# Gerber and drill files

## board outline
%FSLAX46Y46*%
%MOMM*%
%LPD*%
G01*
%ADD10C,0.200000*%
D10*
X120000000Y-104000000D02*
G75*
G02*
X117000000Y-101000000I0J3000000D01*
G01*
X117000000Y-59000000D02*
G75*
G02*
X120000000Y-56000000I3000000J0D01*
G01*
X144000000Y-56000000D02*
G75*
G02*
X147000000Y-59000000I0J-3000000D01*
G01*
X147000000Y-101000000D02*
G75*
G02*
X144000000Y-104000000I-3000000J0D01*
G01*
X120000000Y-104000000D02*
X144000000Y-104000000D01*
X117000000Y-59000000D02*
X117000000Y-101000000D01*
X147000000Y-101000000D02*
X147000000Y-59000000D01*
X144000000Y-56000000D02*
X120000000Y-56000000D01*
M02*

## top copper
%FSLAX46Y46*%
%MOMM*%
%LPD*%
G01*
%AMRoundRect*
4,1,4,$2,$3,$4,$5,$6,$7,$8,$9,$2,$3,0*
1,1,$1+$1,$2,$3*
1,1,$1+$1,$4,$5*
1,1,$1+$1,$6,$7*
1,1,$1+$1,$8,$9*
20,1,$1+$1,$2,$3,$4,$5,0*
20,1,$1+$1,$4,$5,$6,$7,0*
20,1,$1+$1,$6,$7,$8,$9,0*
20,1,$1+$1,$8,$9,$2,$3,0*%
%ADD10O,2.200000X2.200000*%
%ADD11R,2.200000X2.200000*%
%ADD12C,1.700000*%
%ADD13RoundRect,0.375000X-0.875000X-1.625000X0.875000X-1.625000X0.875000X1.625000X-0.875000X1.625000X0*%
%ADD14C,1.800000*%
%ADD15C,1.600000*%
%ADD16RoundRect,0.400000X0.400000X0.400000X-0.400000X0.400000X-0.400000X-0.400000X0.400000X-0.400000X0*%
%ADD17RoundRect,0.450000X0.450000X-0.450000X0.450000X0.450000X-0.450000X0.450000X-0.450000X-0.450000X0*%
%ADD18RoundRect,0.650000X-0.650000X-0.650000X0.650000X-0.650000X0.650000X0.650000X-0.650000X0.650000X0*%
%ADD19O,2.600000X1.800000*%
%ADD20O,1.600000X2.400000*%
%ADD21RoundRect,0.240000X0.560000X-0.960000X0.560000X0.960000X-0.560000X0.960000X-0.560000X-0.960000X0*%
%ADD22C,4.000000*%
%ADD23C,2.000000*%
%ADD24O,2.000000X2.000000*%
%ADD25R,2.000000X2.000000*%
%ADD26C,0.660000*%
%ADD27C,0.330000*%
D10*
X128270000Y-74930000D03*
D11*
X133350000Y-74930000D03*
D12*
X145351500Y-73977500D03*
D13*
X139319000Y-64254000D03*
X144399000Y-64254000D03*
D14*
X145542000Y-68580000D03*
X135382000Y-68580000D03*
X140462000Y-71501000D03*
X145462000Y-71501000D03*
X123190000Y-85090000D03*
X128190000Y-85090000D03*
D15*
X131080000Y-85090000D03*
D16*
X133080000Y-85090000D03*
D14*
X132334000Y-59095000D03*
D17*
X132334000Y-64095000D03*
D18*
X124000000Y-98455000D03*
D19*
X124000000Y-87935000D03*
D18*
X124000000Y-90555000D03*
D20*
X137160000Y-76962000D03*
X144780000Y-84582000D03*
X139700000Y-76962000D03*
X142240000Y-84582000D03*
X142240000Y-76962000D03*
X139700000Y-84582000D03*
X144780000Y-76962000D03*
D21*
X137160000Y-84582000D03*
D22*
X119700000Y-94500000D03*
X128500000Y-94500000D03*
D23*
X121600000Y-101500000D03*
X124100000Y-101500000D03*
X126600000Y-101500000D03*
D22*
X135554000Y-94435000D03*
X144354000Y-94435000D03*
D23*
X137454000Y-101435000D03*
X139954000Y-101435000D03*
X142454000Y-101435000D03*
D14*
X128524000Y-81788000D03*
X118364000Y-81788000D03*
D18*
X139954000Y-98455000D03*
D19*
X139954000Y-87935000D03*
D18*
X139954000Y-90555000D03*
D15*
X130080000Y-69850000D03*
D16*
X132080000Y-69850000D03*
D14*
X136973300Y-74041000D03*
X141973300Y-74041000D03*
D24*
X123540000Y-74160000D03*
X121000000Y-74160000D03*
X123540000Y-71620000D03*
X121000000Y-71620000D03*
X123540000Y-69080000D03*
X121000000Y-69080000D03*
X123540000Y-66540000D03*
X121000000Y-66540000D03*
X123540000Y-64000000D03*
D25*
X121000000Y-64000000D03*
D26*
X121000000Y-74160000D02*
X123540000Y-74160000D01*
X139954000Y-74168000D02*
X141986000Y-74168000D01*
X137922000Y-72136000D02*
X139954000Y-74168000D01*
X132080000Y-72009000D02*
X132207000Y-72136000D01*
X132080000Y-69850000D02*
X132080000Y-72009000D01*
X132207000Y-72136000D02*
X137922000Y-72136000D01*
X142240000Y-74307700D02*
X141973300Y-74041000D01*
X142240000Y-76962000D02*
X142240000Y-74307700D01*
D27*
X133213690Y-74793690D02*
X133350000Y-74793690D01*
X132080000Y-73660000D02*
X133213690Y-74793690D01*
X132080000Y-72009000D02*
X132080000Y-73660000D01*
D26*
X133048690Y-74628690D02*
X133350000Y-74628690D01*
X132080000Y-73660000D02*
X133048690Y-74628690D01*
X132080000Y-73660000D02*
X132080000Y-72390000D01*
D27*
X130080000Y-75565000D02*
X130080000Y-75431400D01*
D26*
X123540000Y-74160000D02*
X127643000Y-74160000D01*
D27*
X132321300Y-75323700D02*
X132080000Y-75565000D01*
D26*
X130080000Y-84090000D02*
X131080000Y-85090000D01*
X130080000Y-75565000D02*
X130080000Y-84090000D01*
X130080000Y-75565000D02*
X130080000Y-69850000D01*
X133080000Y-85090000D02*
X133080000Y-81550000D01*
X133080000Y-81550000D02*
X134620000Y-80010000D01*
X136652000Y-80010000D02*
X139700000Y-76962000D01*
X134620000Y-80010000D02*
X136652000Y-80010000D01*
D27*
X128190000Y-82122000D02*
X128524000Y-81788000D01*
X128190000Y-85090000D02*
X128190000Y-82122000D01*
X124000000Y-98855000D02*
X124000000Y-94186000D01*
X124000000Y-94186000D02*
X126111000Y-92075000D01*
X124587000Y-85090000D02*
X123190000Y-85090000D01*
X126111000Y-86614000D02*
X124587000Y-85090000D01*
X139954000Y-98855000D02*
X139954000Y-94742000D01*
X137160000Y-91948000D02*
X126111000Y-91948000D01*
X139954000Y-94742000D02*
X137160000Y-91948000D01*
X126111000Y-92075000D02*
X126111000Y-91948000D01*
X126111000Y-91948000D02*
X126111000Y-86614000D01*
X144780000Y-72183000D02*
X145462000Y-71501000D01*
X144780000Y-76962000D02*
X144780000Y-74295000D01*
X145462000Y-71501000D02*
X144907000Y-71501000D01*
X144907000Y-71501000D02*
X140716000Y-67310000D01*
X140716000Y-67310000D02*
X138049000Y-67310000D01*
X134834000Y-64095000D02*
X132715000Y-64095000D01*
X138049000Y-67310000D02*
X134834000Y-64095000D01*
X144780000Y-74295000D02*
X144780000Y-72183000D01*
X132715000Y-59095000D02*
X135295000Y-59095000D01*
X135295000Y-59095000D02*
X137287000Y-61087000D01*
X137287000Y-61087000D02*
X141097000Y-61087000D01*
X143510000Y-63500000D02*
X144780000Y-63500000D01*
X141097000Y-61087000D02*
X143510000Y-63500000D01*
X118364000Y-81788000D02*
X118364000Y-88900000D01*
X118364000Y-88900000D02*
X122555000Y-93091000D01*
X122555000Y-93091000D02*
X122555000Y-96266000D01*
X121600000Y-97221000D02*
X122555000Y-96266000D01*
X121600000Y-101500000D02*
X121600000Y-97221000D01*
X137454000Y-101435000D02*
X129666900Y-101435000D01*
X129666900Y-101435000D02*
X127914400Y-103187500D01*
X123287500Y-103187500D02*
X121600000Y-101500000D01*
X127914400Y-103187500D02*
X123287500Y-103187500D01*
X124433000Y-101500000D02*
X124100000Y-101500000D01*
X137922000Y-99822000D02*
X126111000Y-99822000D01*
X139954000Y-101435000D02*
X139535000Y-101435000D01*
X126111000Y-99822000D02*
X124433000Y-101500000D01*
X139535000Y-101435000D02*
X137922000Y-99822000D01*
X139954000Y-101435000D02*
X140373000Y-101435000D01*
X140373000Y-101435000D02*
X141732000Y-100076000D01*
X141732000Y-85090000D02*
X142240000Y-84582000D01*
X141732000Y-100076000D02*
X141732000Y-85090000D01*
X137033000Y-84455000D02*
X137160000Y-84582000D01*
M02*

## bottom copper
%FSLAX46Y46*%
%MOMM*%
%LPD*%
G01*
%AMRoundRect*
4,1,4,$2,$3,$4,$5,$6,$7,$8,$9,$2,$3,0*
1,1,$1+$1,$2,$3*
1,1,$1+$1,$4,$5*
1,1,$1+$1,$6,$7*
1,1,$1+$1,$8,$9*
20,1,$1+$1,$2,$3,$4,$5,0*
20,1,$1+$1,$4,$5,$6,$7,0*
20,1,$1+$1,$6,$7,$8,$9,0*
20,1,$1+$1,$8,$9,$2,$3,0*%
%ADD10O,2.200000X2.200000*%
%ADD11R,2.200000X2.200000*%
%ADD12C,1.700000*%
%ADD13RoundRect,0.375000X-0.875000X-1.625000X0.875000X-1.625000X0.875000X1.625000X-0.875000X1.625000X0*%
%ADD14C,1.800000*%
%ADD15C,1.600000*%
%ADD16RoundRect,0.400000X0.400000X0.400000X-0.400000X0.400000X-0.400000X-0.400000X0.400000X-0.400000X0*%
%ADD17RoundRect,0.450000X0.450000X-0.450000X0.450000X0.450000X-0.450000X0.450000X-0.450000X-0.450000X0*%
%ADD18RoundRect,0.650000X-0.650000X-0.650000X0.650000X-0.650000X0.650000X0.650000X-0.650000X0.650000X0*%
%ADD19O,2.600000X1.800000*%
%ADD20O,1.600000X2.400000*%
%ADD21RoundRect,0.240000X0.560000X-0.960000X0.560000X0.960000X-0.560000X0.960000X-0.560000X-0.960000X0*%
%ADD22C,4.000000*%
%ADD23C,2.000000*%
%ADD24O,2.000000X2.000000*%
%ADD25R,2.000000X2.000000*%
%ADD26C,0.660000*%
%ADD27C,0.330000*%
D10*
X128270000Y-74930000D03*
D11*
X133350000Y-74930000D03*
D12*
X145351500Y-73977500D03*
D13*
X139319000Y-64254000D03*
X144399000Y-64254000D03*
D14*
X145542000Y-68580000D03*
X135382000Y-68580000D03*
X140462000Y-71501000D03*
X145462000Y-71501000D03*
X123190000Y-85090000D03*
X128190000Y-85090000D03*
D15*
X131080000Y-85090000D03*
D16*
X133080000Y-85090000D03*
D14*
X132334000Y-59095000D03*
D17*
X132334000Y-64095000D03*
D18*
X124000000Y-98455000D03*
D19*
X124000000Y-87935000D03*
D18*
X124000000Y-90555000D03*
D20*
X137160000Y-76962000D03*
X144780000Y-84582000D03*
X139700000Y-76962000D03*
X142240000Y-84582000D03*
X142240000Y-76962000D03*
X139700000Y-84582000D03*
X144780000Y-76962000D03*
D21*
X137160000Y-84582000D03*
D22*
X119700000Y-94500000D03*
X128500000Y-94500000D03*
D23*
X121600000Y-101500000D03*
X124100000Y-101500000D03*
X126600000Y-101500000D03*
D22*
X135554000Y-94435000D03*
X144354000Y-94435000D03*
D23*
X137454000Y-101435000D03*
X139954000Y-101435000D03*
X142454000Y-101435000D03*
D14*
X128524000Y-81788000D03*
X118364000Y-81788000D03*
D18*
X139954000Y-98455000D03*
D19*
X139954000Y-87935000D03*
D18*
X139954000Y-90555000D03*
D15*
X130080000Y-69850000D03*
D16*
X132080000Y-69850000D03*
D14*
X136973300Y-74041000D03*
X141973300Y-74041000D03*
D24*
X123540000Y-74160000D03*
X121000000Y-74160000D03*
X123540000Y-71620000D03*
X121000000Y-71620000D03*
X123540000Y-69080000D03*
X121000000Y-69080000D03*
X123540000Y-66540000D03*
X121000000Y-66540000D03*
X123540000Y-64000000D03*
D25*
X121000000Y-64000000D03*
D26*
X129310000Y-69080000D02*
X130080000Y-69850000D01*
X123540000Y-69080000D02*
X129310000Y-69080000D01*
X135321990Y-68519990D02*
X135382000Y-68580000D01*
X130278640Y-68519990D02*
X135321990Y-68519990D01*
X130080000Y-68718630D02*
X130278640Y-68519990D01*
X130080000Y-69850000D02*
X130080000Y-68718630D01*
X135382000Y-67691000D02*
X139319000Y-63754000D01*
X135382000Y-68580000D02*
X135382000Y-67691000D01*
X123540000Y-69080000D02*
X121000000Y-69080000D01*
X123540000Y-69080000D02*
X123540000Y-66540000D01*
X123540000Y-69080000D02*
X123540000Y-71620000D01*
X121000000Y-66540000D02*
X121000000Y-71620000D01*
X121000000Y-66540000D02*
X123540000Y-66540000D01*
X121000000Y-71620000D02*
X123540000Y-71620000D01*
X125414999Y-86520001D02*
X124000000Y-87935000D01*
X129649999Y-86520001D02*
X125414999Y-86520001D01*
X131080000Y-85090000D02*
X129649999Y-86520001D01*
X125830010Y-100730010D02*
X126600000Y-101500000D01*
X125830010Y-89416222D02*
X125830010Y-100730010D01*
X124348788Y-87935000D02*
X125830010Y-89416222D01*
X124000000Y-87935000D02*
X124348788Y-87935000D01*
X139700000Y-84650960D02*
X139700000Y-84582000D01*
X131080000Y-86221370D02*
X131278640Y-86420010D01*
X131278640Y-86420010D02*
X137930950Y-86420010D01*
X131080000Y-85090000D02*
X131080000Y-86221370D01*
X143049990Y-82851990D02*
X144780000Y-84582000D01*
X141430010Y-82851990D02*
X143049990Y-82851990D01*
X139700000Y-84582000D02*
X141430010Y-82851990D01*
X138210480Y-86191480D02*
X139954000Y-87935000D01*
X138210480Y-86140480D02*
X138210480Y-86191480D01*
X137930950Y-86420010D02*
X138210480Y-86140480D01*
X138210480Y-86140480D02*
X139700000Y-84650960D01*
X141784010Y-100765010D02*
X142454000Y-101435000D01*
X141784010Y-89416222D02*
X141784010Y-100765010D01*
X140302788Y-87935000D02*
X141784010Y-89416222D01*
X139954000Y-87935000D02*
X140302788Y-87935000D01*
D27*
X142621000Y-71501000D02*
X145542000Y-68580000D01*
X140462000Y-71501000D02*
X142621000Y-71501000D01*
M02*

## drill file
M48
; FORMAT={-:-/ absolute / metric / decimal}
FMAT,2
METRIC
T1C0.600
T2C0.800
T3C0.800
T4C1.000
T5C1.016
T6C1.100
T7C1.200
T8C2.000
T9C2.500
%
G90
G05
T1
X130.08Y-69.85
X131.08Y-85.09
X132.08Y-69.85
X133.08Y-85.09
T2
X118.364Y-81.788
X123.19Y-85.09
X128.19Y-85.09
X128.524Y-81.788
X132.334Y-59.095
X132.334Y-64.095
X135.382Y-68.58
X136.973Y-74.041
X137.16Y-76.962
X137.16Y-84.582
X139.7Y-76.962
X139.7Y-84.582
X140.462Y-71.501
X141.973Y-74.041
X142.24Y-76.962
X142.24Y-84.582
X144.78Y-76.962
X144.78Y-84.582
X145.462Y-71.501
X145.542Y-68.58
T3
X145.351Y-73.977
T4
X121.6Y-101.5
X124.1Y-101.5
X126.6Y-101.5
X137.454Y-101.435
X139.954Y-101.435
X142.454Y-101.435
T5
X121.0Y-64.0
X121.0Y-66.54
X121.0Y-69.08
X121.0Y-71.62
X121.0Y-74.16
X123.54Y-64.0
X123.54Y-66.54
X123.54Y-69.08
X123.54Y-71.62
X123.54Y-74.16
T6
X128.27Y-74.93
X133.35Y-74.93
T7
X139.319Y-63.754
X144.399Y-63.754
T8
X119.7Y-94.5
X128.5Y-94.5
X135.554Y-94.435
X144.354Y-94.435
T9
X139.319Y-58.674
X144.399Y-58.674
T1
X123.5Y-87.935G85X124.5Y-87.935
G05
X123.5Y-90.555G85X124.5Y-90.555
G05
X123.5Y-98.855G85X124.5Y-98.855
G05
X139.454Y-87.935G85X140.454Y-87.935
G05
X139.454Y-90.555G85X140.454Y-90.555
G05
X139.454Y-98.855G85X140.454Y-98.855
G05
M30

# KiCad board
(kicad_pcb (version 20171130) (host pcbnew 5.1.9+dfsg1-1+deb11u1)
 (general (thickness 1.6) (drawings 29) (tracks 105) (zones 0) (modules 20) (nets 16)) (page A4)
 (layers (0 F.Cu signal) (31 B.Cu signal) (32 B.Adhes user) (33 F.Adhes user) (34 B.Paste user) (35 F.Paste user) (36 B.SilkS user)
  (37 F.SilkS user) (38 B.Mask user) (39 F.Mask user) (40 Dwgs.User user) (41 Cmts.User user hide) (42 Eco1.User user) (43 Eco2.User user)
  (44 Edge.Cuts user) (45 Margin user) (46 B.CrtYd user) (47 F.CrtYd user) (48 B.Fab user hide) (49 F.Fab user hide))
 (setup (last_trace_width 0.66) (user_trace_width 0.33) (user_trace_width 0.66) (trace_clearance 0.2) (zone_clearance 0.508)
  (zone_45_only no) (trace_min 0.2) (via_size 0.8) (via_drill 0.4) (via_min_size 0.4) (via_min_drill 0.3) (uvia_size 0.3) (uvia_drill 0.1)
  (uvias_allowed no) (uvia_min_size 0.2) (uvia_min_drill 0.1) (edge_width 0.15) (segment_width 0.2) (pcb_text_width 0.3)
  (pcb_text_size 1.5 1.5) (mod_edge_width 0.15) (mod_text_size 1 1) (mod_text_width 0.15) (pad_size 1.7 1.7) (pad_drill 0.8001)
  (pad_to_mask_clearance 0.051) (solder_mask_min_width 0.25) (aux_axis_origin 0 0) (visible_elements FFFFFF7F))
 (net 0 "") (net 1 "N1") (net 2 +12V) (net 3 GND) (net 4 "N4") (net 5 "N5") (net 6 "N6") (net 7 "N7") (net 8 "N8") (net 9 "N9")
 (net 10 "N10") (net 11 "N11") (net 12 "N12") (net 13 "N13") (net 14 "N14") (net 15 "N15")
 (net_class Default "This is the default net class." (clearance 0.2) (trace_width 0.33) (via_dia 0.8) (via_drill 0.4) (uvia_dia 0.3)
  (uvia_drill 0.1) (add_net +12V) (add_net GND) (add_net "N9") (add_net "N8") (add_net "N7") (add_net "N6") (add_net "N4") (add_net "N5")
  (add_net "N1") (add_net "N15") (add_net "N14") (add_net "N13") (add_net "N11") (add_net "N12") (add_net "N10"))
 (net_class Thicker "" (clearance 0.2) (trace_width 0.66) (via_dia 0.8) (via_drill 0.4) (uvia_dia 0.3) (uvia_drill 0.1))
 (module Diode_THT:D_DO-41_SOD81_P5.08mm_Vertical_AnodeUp (layer F.Cu) (at 133.35 74.93 180)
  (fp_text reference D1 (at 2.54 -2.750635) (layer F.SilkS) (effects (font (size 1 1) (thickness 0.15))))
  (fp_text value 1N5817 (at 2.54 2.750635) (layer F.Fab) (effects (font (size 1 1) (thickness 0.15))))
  (pad 2 thru_hole oval (at 5.08 0 180) (size 2.2 2.2) (drill 1.1) (layers *.Cu *.Mask) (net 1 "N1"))
  (pad 1 thru_hole rect (at 0 0 180) (size 2.2 2.2) (drill 1.1) (layers *.Cu *.Mask) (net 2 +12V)))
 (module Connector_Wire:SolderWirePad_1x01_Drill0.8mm (layer F.Cu) (at 145.3515 73.9775)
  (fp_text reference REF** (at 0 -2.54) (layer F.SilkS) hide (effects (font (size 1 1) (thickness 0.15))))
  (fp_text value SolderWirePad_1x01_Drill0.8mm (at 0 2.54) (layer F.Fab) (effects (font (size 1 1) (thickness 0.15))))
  (pad 1 thru_hole circle (at 0 0) (size 1.7 1.7) (drill 0.8001) (layers *.Cu *.Mask)))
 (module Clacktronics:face (layer B.Cu) (at 140.843 80.772 180)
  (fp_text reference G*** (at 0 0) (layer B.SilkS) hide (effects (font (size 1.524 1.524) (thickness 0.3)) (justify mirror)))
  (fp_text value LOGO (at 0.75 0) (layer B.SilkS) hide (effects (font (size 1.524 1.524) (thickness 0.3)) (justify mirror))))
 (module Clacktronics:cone (layer B.Cu) (at 122.047 60.579 180)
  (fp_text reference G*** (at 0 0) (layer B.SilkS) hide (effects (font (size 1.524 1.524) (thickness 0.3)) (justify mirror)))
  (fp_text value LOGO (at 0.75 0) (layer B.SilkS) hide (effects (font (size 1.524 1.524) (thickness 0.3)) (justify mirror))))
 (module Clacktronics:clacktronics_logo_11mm (layer F.Cu) (at 131.572 87.63)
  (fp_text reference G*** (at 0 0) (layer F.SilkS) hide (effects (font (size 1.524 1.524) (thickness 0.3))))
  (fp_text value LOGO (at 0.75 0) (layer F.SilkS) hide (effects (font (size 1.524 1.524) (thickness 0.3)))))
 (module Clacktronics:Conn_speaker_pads (layer F.Cu) (at 141.859 63.754)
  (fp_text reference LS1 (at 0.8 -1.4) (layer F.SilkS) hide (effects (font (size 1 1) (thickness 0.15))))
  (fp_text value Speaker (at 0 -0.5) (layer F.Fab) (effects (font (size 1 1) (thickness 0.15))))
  (pad 2 thru_hole roundrect (at -2.54 0) (size 2.5 4) (drill 1.2 (offset 0 0.5)) (layers *.Cu *.Mask) (roundrect_rratio 0.15) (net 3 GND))
  (pad "" np_thru_hole circle (at -2.54 -5.08) (size 2.5 2.5) (drill 2.5) (layers *.Cu *.Mask))
  (pad 1 thru_hole roundrect (at 2.54 0) (size 2.5 4) (drill 1.2 (offset 0 0.5)) (layers *.Cu *.Mask) (roundrect_rratio 0.15) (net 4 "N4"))
  (pad "" np_thru_hole circle (at 2.54 -5.08) (size 2.5 2.5) (drill 2.5) (layers *.Cu *.Mask)))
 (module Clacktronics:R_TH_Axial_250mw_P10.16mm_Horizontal (layer F.Cu) (at 135.382 68.58)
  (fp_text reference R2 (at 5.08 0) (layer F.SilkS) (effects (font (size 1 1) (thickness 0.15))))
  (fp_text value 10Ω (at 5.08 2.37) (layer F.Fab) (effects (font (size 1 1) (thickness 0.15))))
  (pad 2 thru_hole circle (at 10.16 0) (size 1.8 1.8) (drill 0.8) (layers *.Cu *.Mask) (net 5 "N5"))
  (pad 1 thru_hole circle (at 0 0) (size 1.8 1.8) (drill 0.8) (layers *.Cu *.Mask) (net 3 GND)))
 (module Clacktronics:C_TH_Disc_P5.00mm (layer F.Cu) (at 145.462 71.501 180)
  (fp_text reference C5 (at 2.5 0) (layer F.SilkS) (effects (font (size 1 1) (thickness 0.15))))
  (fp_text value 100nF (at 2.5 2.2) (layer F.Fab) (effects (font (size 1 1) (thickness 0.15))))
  (pad 2 thru_hole circle (at 5 0 180) (size 1.8 1.8) (drill 0.8) (layers *.Cu *.Mask) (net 5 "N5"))
  (pad 1 thru_hole circle (at 0 0 180) (size 1.8 1.8) (drill 0.8) (layers *.Cu *.Mask) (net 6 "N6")))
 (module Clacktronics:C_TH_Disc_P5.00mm (layer F.Cu) (at 128.19 85.09 180)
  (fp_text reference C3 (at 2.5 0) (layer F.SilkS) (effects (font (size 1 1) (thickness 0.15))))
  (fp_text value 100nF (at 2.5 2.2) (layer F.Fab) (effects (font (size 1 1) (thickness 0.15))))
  (pad 2 thru_hole circle (at 5 0 180) (size 1.8 1.8) (drill 0.8) (layers *.Cu *.Mask) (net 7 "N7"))
  (pad 1 thru_hole circle (at 0 0 180) (size 1.8 1.8) (drill 0.8) (layers *.Cu *.Mask) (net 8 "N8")))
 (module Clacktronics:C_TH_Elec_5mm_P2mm (layer F.Cu) (at 132.08 85.09 180)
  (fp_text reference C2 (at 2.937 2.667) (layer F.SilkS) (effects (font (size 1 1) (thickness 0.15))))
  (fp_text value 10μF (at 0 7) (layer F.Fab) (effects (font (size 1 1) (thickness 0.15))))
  (pad 2 thru_hole circle (at 1 0 180) (size 1.6 1.6) (drill 0.6) (layers *.Cu *.Mask) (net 3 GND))
  (pad 1 thru_hole roundrect (at -1 0 180) (size 1.6 1.6) (drill 0.6) (layers *.Cu *.Mask) (roundrect_rratio 0.25) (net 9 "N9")))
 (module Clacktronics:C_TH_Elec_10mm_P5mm (layer F.Cu) (at 132.334 61.595 90)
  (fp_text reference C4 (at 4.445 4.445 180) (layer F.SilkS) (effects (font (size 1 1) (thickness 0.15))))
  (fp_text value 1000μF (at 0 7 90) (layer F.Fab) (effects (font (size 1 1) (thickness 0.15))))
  (pad 2 thru_hole circle (at 2.5 0 90) (size 1.8 1.8) (drill 0.8) (layers *.Cu *.Mask) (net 4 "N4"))
  (pad 1 thru_hole roundrect (at -2.5 0 90) (size 1.8 1.8) (drill 0.8) (layers *.Cu *.Mask) (roundrect_rratio 0.25) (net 6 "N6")))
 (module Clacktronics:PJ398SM (layer B.Cu) (at 124 93.935 180)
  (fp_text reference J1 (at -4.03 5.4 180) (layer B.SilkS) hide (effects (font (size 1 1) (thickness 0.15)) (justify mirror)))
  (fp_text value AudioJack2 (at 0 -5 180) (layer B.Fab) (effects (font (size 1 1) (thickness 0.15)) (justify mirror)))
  (pad T thru_hole roundrect (at 0 -4.92) (size 2.6 2.6) (drill oval 1.6 0.6 (offset 0 -0.4)) (layers *.Cu *.Mask) (roundrect_rratio 0.25)
   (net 7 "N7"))
  (pad S thru_hole oval (at 0 6) (size 2.6 1.8) (drill oval 1.6 0.6) (layers *.Cu *.Mask) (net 3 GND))
  (pad TN thru_hole roundrect (at 0 3.38) (size 2.6 2.6) (drill oval 1.6 0.6) (layers *.Cu *.Mask) (roundrect_rratio 0.25)))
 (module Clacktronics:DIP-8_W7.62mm (layer F.Cu) (at 137.16 84.582 90)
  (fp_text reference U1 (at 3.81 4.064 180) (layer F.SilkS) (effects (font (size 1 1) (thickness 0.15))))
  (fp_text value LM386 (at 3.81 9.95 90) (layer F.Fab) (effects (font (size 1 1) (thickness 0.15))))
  (pad 8 thru_hole oval (at 7.62 0 90) (size 2.4 1.6) (drill 0.8) (layers *.Cu *.Mask) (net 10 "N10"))
  (pad 4 thru_hole oval (at 0 7.62 90) (size 2.4 1.6) (drill 0.8) (layers *.Cu *.Mask) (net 3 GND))
  (pad 7 thru_hole oval (at 7.62 2.54 90) (size 2.4 1.6) (drill 0.8) (layers *.Cu *.Mask) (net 9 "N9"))
  (pad 3 thru_hole oval (at 0 5.08 90) (size 2.4 1.6) (drill 0.8) (layers *.Cu *.Mask) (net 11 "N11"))
  (pad 6 thru_hole oval (at 7.62 5.08 90) (size 2.4 1.6) (drill 0.8) (layers *.Cu *.Mask) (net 2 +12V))
  (pad 2 thru_hole oval (at 0 2.54 90) (size 2.4 1.6) (drill 0.8) (layers *.Cu *.Mask) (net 3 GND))
  (pad 5 thru_hole oval (at 7.62 7.62 90) (size 2.4 1.6) (drill 0.8) (layers *.Cu *.Mask) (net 6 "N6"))
  (pad 1 thru_hole roundrect (at 0 0 90) (size 2.4 1.6) (drill 0.8) (layers *.Cu *.Mask) (roundrect_rratio 0.15) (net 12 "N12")))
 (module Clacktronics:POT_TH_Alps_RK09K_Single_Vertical (layer B.Cu) (at 124.1 94 180)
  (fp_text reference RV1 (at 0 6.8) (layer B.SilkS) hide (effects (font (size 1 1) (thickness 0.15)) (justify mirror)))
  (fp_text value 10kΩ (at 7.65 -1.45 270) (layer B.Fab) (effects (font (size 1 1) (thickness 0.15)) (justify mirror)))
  (pad "" thru_hole circle (at 4.4 -0.5 90) (size 4 4) (drill 2) (layers *.Cu *.Mask))
  (pad "" thru_hole circle (at -4.4 -0.5 90) (size 4 4) (drill 2) (layers *.Cu *.Mask))
  (pad 1 thru_hole circle (at 2.5 -7.5 90) (size 2 2) (drill 1) (layers *.Cu *.Mask) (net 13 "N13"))
  (pad 2 thru_hole circle (at 0 -7.5 180) (size 2 2) (drill 1) (layers *.Cu *.Mask) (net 11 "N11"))
  (pad 3 thru_hole circle (at -2.5 -7.5 90) (size 2 2) (drill 1) (layers *.Cu *.Mask) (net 3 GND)))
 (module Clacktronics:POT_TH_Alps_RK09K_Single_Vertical (layer B.Cu) (at 139.954 93.935 180)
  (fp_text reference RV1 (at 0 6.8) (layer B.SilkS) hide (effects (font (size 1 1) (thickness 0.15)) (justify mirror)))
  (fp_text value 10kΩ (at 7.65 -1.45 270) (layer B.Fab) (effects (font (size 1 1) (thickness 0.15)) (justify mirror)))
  (pad "" thru_hole circle (at 4.4 -0.5 90) (size 4 4) (drill 2) (layers *.Cu *.Mask))
  (pad "" thru_hole circle (at -4.4 -0.5 90) (size 4 4) (drill 2) (layers *.Cu *.Mask))
  (pad 1 thru_hole circle (at 2.5 -7.5 90) (size 2 2) (drill 1) (layers *.Cu *.Mask) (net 13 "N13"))
  (pad 2 thru_hole circle (at 0 -7.5 180) (size 2 2) (drill 1) (layers *.Cu *.Mask) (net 11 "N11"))
  (pad 3 thru_hole circle (at -2.5 -7.5 90) (size 2 2) (drill 1) (layers *.Cu *.Mask) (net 3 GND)))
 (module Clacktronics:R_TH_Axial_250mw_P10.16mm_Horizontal (layer F.Cu) (at 118.364 81.788)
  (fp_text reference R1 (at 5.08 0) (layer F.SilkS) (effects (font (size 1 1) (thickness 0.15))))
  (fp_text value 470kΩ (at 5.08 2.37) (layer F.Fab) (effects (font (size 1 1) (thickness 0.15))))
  (pad 2 thru_hole circle (at 10.16 0) (size 1.8 1.8) (drill 0.8) (layers *.Cu *.Mask) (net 8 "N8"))
  (pad 1 thru_hole circle (at 0 0) (size 1.8 1.8) (drill 0.8) (layers *.Cu *.Mask) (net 13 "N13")))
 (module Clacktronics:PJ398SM (layer B.Cu) (at 139.954 93.935 180)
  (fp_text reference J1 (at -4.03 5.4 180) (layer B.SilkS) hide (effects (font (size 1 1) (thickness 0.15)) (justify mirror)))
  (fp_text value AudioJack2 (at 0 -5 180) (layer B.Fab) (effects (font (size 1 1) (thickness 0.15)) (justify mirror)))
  (pad T thru_hole roundrect (at 0 -4.92) (size 2.6 2.6) (drill oval 1.6 0.6 (offset 0 -0.4)) (layers *.Cu *.Mask) (roundrect_rratio 0.25)
   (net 7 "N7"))
  (pad S thru_hole oval (at 0 6) (size 2.6 1.8) (drill oval 1.6 0.6) (layers *.Cu *.Mask) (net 3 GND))
  (pad TN thru_hole roundrect (at 0 3.38) (size 2.6 2.6) (drill oval 1.6 0.6) (layers *.Cu *.Mask) (roundrect_rratio 0.25)))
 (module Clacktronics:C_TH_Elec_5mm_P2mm (layer F.Cu) (at 131.08 69.85 180)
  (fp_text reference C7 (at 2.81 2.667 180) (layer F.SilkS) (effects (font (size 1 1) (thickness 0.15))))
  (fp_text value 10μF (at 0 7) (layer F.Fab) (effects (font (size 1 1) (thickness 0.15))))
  (pad 2 thru_hole circle (at 1 0 180) (size 1.6 1.6) (drill 0.6) (layers *.Cu *.Mask) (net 3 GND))
  (pad 1 thru_hole roundrect (at -1 0 180) (size 1.6 1.6) (drill 0.6) (layers *.Cu *.Mask) (roundrect_rratio 0.25) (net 2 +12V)))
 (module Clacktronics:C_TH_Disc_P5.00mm (layer F.Cu) (at 141.9733 74.041 180)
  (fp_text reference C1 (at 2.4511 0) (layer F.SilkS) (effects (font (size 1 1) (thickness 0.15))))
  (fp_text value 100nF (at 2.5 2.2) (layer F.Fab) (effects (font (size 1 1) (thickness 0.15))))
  (pad 2 thru_hole circle (at 5 0 180) (size 1.8 1.8) (drill 0.8) (layers *.Cu *.Mask) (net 3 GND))
  (pad 1 thru_hole circle (at 0 0 180) (size 1.8 1.8) (drill 0.8) (layers *.Cu *.Mask) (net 2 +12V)))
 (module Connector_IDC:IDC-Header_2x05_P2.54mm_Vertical (layer F.Cu) (at 121 64)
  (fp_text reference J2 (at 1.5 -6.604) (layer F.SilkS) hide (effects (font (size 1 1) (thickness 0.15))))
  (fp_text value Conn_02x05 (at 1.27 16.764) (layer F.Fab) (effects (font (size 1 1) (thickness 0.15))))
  (pad 10 thru_hole oval (at 2.54 10.16) (size 2 2) (drill 1.016) (layers *.Cu *.Mask) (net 1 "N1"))
  (pad 9 thru_hole oval (at 0 10.16) (size 2 2) (drill 1.016) (layers *.Cu *.Mask) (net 1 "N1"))
  (pad 8 thru_hole oval (at 2.54 7.62) (size 2 2) (drill 1.016) (layers *.Cu *.Mask) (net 3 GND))
  (pad 7 thru_hole oval (at 0 7.62) (size 2 2) (drill 1.016) (layers *.Cu *.Mask) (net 3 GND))
  (pad 6 thru_hole oval (at 2.54 5.08) (size 2 2) (drill 1.016) (layers *.Cu *.Mask) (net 3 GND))
  (pad 5 thru_hole oval (at 0 5.08) (size 2 2) (drill 1.016) (layers *.Cu *.Mask) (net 3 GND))
  (pad 4 thru_hole oval (at 2.54 2.54) (size 2 2) (drill 1.016) (layers *.Cu *.Mask) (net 3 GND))
  (pad 3 thru_hole oval (at 0 2.54) (size 2 2) (drill 1.016) (layers *.Cu *.Mask) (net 3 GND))
  (pad 2 thru_hole oval (at 2.54 0) (size 2 2) (drill 1.016) (layers *.Cu *.Mask) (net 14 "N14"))
  (pad 1 thru_hole rect (at 0 0) (size 2 2) (drill 1.016) (layers *.Cu *.Mask) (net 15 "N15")))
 (gr_arc (start 120 101) (end 117 101) (angle -90) (layer Edge.Cuts) (width 0.2))
 (gr_arc (start 120 59) (end 120 56) (angle -90) (layer Edge.Cuts) (width 0.2))
 (gr_arc (start 144 59) (end 147 59) (angle -90) (layer Edge.Cuts) (width 0.2))
 (gr_arc (start 144 101) (end 144 104) (angle -90) (layer Edge.Cuts) (width 0.2))
 (gr_line (start 120 104) (end 144 104) (layer Edge.Cuts) (width 0.2))
 (gr_line (start 117 59) (end 117 101) (layer Edge.Cuts) (width 0.2))
 (gr_line (start 147 101) (end 147 59) (layer Edge.Cuts) (width 0.2))
 (gr_line (start 144 56) (end 120 56) (layer Edge.Cuts) (width 0.2))
 (segment (start 121 74.16) (end 123.54 74.16) (width 0.66) (layer F.Cu) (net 1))
 (segment (start 139.954 74.168) (end 141.986 74.168) (width 0.66) (layer F.Cu) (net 2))
 (segment (start 137.922 72.136) (end 139.954 74.168) (width 0.66) (layer F.Cu) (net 2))
 (segment (start 132.08 72.009) (end 132.207 72.136) (width 0.66) (layer F.Cu) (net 2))
 (segment (start 132.08 69.85) (end 132.08 72.009) (width 0.66) (layer F.Cu) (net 2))
 (segment (start 132.207 72.136) (end 137.922 72.136) (width 0.66) (layer F.Cu) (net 2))
 (segment (start 142.24 74.3077) (end 141.9733 74.041) (width 0.66) (layer F.Cu) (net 2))
 (segment (start 142.24 76.962) (end 142.24 74.3077) (width 0.66) (layer F.Cu) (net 2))
 (segment (start 133.21369 74.79369) (end 133.35 74.79369) (width 0.33) (layer F.Cu) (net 2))
 (segment (start 132.08 73.66) (end 133.21369 74.79369) (width 0.33) (layer F.Cu) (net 2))
 (segment (start 132.08 72.009) (end 132.08 73.66) (width 0.33) (layer F.Cu) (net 2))
 (segment (start 133.04869 74.62869) (end 133.35 74.62869) (width 0.66) (layer F.Cu) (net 2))
 (segment (start 132.08 73.66) (end 133.04869 74.62869) (width 0.66) (layer F.Cu) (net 2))
 (segment (start 132.08 73.66) (end 132.08 72.39) (width 0.66) (layer F.Cu) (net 2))
 (segment (start 130.08 75.565) (end 130.08 75.4314) (width 0.33) (layer F.Cu) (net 3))
 (segment (start 123.54 74.16) (end 127.643 74.16) (width 0.66) (layer F.Cu) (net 1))
 (segment (start 132.3213 75.3237) (end 132.08 75.565) (width 0.33) (layer F.Cu) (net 2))
 (segment (start 129.31 69.08) (end 130.08 69.85) (width 0.66) (layer B.Cu) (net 3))
 (segment (start 123.54 69.08) (end 129.31 69.08) (width 0.66) (layer B.Cu) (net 3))
 (segment (start 135.32199 68.51999) (end 135.382 68.58) (width 0.66) (layer B.Cu) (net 3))
 (segment (start 130.27864 68.51999) (end 135.32199 68.51999) (width 0.66) (layer B.Cu) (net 3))
 (segment (start 130.08 68.71863) (end 130.27864 68.51999) (width 0.66) (layer B.Cu) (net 3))
 (segment (start 130.08 69.85) (end 130.08 68.71863) (width 0.66) (layer B.Cu) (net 3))
 (segment (start 135.382 67.691) (end 139.319 63.754) (width 0.66) (layer B.Cu) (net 3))
 (segment (start 135.382 68.58) (end 135.382 67.691) (width 0.66) (layer B.Cu) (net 3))
 (segment (start 123.54 69.08) (end 121 69.08) (width 0.66) (layer B.Cu) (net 3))
 (segment (start 123.54 69.08) (end 123.54 66.54) (width 0.66) (layer B.Cu) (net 3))
 (segment (start 123.54 69.08) (end 123.54 71.62) (width 0.66) (layer B.Cu) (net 3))
 (segment (start 121 66.54) (end 121 71.62) (width 0.66) (layer B.Cu) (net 3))
 (segment (start 121 66.54) (end 123.54 66.54) (width 0.66) (layer B.Cu) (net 3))
 (segment (start 121 71.62) (end 123.54 71.62) (width 0.66) (layer B.Cu) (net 3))
 (segment (start 130.08 84.09) (end 131.08 85.09) (width 0.66) (layer F.Cu) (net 3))
 (segment (start 130.08 75.565) (end 130.08 84.09) (width 0.66) (layer F.Cu) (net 3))
 (segment (start 130.08 75.565) (end 130.08 69.85) (width 0.66) (layer F.Cu) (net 3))
 (segment (start 125.414999 86.520001) (end 124 87.935) (width 0.66) (layer B.Cu) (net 3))
 (segment (start 129.649999 86.520001) (end 125.414999 86.520001) (width 0.66) (layer B.Cu) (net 3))
 (segment (start 131.08 85.09) (end 129.649999 86.520001) (width 0.66) (layer B.Cu) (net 3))
 (segment (start 125.83001 100.73001) (end 126.6 101.5) (width 0.66) (layer B.Cu) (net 3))
 (segment (start 125.83001 89.416222) (end 125.83001 100.73001) (width 0.66) (layer B.Cu) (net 3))
 (segment (start 124.348788 87.935) (end 125.83001 89.416222) (width 0.66) (layer B.Cu) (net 3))
 (segment (start 124 87.935) (end 124.348788 87.935) (width 0.66) (layer B.Cu) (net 3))
 (segment (start 139.7 84.65096) (end 139.7 84.582) (width 0.66) (layer B.Cu) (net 3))
 (segment (start 131.08 86.22137) (end 131.27864 86.42001) (width 0.66) (layer B.Cu) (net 3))
 (segment (start 131.27864 86.42001) (end 137.93095 86.42001) (width 0.66) (layer B.Cu) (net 3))
 (segment (start 131.08 85.09) (end 131.08 86.22137) (width 0.66) (layer B.Cu) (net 3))
 (segment (start 143.04999 82.85199) (end 144.78 84.582) (width 0.66) (layer B.Cu) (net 3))
 (segment (start 141.43001 82.85199) (end 143.04999 82.85199) (width 0.66) (layer B.Cu) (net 3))
 (segment (start 139.7 84.582) (end 141.43001 82.85199) (width 0.66) (layer B.Cu) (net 3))
 (segment (start 138.21048 86.19148) (end 139.954 87.935) (width 0.66) (layer B.Cu) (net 3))
 (segment (start 138.21048 86.14048) (end 138.21048 86.19148) (width 0.66) (layer B.Cu) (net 3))
 (segment (start 137.93095 86.42001) (end 138.21048 86.14048) (width 0.66) (layer B.Cu) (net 3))
 (segment (start 138.21048 86.14048) (end 139.7 84.65096) (width 0.66) (layer B.Cu) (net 3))
 (segment (start 141.78401 100.76501) (end 142.454 101.435) (width 0.66) (layer B.Cu) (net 3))
 (segment (start 141.78401 89.416222) (end 141.78401 100.76501) (width 0.66) (layer B.Cu) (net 3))
 (segment (start 140.302788 87.935) (end 141.78401 89.416222) (width 0.66) (layer B.Cu) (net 3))
 (segment (start 139.954 87.935) (end 140.302788 87.935) (width 0.66) (layer B.Cu) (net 3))
 (segment (start 133.08 85.09) (end 133.08 81.55) (width 0.66) (layer F.Cu) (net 9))
 (segment (start 133.08 81.55) (end 134.62 80.01) (width 0.66) (layer F.Cu) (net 9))
 (segment (start 136.652 80.01) (end 139.7 76.962) (width 0.66) (layer F.Cu) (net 9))
 (segment (start 134.62 80.01) (end 136.652 80.01) (width 0.66) (layer F.Cu) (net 9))
 (segment (start 128.19 82.122) (end 128.524 81.788) (width 0.33) (layer F.Cu) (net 8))
 (segment (start 128.19 85.09) (end 128.19 82.122) (width 0.33) (layer F.Cu) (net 8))
 (segment (start 124 98.855) (end 124 94.186) (width 0.33) (layer F.Cu) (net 7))
 (segment (start 124 94.186) (end 126.111 92.075) (width 0.33) (layer F.Cu) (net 7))
 (segment (start 124.587 85.09) (end 123.19 85.09) (width 0.33) (layer F.Cu) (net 7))
 (segment (start 126.111 86.614) (end 124.587 85.09) (width 0.33) (layer F.Cu) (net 7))
 (segment (start 139.954 98.855) (end 139.954 94.742) (width 0.33) (layer F.Cu) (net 7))
 (segment (start 137.16 91.948) (end 126.111 91.948) (width 0.33) (layer F.Cu) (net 7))
 (segment (start 139.954 94.742) (end 137.16 91.948) (width 0.33) (layer F.Cu) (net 7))
 (segment (start 126.111 92.075) (end 126.111 91.948) (width 0.33) (layer F.Cu) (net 7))
 (segment (start 126.111 91.948) (end 126.111 86.614) (width 0.33) (layer F.Cu) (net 7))
 (segment (start 144.78 72.183) (end 145.462 71.501) (width 0.33) (layer F.Cu) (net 6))
 (segment (start 144.78 76.962) (end 144.78 74.295) (width 0.33) (layer F.Cu) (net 6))
 (segment (start 145.462 71.501) (end 144.907 71.501) (width 0.33) (layer F.Cu) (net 6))
 (segment (start 144.907 71.501) (end 140.716 67.31) (width 0.33) (layer F.Cu) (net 6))
 (segment (start 140.716 67.31) (end 138.049 67.31) (width 0.33) (layer F.Cu) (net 6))
 (segment (start 134.834 64.095) (end 132.715 64.095) (width 0.33) (layer F.Cu) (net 6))
 (segment (start 138.049 67.31) (end 134.834 64.095) (width 0.33) (layer F.Cu) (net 6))
 (segment (start 144.78 74.295) (end 144.78 72.183) (width 0.33) (layer F.Cu) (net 6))
 (segment (start 132.715 59.095) (end 135.295 59.095) (width 0.33) (layer F.Cu) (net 4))
 (segment (start 135.295 59.095) (end 137.287 61.087) (width 0.33) (layer F.Cu) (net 4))
 (segment (start 137.287 61.087) (end 141.097 61.087) (width 0.33) (layer F.Cu) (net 4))
 (segment (start 143.51 63.5) (end 144.78 63.5) (width 0.33) (layer F.Cu) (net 4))
 (segment (start 141.097 61.087) (end 143.51 63.5) (width 0.33) (layer F.Cu) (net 4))
 (segment (start 118.364 81.788) (end 118.364 88.9) (width 0.33) (layer F.Cu) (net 13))
 (segment (start 118.364 88.9) (end 122.555 93.091) (width 0.33) (layer F.Cu) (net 13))
 (segment (start 122.555 93.091) (end 122.555 96.266) (width 0.33) (layer F.Cu) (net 13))
 (segment (start 121.6 97.221) (end 122.555 96.266) (width 0.33) (layer F.Cu) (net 13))
 (segment (start 121.6 101.5) (end 121.6 97.221) (width 0.33) (layer F.Cu) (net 13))
 (segment (start 137.454 101.435) (end 129.6669 101.435) (width 0.33) (layer F.Cu) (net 13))
 (segment (start 129.6669 101.435) (end 127.9144 103.1875) (width 0.33) (layer F.Cu) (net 13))
 (segment (start 123.2875 103.1875) (end 121.6 101.5) (width 0.33) (layer F.Cu) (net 13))
 (segment (start 127.9144 103.1875) (end 123.2875 103.1875) (width 0.33) (layer F.Cu) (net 13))
 (segment (start 124.433 101.5) (end 124.1 101.5) (width 0.33) (layer F.Cu) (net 11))
 (segment (start 137.922 99.822) (end 126.111 99.822) (width 0.33) (layer F.Cu) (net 11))
 (segment (start 139.954 101.435) (end 139.535 101.435) (width 0.33) (layer F.Cu) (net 11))
 (segment (start 126.111 99.822) (end 124.433 101.5) (width 0.33) (layer F.Cu) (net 11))
 (segment (start 139.535 101.435) (end 137.922 99.822) (width 0.33) (layer F.Cu) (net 11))
 (segment (start 139.954 101.435) (end 140.373 101.435) (width 0.33) (layer F.Cu) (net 11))
 (segment (start 140.373 101.435) (end 141.732 100.076) (width 0.33) (layer F.Cu) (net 11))
 (segment (start 141.732 85.09) (end 142.24 84.582) (width 0.33) (layer F.Cu) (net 11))
 (segment (start 141.732 100.076) (end 141.732 85.09) (width 0.33) (layer F.Cu) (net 11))
 (segment (start 142.621 71.501) (end 145.542 68.58) (width 0.33) (layer B.Cu) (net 5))
 (segment (start 140.462 71.501) (end 142.621 71.501) (width 0.33) (layer B.Cu) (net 5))
 (segment (start 137.033 84.455) (end 137.16 84.582) (width 0.33) (layer F.Cu) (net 12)))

